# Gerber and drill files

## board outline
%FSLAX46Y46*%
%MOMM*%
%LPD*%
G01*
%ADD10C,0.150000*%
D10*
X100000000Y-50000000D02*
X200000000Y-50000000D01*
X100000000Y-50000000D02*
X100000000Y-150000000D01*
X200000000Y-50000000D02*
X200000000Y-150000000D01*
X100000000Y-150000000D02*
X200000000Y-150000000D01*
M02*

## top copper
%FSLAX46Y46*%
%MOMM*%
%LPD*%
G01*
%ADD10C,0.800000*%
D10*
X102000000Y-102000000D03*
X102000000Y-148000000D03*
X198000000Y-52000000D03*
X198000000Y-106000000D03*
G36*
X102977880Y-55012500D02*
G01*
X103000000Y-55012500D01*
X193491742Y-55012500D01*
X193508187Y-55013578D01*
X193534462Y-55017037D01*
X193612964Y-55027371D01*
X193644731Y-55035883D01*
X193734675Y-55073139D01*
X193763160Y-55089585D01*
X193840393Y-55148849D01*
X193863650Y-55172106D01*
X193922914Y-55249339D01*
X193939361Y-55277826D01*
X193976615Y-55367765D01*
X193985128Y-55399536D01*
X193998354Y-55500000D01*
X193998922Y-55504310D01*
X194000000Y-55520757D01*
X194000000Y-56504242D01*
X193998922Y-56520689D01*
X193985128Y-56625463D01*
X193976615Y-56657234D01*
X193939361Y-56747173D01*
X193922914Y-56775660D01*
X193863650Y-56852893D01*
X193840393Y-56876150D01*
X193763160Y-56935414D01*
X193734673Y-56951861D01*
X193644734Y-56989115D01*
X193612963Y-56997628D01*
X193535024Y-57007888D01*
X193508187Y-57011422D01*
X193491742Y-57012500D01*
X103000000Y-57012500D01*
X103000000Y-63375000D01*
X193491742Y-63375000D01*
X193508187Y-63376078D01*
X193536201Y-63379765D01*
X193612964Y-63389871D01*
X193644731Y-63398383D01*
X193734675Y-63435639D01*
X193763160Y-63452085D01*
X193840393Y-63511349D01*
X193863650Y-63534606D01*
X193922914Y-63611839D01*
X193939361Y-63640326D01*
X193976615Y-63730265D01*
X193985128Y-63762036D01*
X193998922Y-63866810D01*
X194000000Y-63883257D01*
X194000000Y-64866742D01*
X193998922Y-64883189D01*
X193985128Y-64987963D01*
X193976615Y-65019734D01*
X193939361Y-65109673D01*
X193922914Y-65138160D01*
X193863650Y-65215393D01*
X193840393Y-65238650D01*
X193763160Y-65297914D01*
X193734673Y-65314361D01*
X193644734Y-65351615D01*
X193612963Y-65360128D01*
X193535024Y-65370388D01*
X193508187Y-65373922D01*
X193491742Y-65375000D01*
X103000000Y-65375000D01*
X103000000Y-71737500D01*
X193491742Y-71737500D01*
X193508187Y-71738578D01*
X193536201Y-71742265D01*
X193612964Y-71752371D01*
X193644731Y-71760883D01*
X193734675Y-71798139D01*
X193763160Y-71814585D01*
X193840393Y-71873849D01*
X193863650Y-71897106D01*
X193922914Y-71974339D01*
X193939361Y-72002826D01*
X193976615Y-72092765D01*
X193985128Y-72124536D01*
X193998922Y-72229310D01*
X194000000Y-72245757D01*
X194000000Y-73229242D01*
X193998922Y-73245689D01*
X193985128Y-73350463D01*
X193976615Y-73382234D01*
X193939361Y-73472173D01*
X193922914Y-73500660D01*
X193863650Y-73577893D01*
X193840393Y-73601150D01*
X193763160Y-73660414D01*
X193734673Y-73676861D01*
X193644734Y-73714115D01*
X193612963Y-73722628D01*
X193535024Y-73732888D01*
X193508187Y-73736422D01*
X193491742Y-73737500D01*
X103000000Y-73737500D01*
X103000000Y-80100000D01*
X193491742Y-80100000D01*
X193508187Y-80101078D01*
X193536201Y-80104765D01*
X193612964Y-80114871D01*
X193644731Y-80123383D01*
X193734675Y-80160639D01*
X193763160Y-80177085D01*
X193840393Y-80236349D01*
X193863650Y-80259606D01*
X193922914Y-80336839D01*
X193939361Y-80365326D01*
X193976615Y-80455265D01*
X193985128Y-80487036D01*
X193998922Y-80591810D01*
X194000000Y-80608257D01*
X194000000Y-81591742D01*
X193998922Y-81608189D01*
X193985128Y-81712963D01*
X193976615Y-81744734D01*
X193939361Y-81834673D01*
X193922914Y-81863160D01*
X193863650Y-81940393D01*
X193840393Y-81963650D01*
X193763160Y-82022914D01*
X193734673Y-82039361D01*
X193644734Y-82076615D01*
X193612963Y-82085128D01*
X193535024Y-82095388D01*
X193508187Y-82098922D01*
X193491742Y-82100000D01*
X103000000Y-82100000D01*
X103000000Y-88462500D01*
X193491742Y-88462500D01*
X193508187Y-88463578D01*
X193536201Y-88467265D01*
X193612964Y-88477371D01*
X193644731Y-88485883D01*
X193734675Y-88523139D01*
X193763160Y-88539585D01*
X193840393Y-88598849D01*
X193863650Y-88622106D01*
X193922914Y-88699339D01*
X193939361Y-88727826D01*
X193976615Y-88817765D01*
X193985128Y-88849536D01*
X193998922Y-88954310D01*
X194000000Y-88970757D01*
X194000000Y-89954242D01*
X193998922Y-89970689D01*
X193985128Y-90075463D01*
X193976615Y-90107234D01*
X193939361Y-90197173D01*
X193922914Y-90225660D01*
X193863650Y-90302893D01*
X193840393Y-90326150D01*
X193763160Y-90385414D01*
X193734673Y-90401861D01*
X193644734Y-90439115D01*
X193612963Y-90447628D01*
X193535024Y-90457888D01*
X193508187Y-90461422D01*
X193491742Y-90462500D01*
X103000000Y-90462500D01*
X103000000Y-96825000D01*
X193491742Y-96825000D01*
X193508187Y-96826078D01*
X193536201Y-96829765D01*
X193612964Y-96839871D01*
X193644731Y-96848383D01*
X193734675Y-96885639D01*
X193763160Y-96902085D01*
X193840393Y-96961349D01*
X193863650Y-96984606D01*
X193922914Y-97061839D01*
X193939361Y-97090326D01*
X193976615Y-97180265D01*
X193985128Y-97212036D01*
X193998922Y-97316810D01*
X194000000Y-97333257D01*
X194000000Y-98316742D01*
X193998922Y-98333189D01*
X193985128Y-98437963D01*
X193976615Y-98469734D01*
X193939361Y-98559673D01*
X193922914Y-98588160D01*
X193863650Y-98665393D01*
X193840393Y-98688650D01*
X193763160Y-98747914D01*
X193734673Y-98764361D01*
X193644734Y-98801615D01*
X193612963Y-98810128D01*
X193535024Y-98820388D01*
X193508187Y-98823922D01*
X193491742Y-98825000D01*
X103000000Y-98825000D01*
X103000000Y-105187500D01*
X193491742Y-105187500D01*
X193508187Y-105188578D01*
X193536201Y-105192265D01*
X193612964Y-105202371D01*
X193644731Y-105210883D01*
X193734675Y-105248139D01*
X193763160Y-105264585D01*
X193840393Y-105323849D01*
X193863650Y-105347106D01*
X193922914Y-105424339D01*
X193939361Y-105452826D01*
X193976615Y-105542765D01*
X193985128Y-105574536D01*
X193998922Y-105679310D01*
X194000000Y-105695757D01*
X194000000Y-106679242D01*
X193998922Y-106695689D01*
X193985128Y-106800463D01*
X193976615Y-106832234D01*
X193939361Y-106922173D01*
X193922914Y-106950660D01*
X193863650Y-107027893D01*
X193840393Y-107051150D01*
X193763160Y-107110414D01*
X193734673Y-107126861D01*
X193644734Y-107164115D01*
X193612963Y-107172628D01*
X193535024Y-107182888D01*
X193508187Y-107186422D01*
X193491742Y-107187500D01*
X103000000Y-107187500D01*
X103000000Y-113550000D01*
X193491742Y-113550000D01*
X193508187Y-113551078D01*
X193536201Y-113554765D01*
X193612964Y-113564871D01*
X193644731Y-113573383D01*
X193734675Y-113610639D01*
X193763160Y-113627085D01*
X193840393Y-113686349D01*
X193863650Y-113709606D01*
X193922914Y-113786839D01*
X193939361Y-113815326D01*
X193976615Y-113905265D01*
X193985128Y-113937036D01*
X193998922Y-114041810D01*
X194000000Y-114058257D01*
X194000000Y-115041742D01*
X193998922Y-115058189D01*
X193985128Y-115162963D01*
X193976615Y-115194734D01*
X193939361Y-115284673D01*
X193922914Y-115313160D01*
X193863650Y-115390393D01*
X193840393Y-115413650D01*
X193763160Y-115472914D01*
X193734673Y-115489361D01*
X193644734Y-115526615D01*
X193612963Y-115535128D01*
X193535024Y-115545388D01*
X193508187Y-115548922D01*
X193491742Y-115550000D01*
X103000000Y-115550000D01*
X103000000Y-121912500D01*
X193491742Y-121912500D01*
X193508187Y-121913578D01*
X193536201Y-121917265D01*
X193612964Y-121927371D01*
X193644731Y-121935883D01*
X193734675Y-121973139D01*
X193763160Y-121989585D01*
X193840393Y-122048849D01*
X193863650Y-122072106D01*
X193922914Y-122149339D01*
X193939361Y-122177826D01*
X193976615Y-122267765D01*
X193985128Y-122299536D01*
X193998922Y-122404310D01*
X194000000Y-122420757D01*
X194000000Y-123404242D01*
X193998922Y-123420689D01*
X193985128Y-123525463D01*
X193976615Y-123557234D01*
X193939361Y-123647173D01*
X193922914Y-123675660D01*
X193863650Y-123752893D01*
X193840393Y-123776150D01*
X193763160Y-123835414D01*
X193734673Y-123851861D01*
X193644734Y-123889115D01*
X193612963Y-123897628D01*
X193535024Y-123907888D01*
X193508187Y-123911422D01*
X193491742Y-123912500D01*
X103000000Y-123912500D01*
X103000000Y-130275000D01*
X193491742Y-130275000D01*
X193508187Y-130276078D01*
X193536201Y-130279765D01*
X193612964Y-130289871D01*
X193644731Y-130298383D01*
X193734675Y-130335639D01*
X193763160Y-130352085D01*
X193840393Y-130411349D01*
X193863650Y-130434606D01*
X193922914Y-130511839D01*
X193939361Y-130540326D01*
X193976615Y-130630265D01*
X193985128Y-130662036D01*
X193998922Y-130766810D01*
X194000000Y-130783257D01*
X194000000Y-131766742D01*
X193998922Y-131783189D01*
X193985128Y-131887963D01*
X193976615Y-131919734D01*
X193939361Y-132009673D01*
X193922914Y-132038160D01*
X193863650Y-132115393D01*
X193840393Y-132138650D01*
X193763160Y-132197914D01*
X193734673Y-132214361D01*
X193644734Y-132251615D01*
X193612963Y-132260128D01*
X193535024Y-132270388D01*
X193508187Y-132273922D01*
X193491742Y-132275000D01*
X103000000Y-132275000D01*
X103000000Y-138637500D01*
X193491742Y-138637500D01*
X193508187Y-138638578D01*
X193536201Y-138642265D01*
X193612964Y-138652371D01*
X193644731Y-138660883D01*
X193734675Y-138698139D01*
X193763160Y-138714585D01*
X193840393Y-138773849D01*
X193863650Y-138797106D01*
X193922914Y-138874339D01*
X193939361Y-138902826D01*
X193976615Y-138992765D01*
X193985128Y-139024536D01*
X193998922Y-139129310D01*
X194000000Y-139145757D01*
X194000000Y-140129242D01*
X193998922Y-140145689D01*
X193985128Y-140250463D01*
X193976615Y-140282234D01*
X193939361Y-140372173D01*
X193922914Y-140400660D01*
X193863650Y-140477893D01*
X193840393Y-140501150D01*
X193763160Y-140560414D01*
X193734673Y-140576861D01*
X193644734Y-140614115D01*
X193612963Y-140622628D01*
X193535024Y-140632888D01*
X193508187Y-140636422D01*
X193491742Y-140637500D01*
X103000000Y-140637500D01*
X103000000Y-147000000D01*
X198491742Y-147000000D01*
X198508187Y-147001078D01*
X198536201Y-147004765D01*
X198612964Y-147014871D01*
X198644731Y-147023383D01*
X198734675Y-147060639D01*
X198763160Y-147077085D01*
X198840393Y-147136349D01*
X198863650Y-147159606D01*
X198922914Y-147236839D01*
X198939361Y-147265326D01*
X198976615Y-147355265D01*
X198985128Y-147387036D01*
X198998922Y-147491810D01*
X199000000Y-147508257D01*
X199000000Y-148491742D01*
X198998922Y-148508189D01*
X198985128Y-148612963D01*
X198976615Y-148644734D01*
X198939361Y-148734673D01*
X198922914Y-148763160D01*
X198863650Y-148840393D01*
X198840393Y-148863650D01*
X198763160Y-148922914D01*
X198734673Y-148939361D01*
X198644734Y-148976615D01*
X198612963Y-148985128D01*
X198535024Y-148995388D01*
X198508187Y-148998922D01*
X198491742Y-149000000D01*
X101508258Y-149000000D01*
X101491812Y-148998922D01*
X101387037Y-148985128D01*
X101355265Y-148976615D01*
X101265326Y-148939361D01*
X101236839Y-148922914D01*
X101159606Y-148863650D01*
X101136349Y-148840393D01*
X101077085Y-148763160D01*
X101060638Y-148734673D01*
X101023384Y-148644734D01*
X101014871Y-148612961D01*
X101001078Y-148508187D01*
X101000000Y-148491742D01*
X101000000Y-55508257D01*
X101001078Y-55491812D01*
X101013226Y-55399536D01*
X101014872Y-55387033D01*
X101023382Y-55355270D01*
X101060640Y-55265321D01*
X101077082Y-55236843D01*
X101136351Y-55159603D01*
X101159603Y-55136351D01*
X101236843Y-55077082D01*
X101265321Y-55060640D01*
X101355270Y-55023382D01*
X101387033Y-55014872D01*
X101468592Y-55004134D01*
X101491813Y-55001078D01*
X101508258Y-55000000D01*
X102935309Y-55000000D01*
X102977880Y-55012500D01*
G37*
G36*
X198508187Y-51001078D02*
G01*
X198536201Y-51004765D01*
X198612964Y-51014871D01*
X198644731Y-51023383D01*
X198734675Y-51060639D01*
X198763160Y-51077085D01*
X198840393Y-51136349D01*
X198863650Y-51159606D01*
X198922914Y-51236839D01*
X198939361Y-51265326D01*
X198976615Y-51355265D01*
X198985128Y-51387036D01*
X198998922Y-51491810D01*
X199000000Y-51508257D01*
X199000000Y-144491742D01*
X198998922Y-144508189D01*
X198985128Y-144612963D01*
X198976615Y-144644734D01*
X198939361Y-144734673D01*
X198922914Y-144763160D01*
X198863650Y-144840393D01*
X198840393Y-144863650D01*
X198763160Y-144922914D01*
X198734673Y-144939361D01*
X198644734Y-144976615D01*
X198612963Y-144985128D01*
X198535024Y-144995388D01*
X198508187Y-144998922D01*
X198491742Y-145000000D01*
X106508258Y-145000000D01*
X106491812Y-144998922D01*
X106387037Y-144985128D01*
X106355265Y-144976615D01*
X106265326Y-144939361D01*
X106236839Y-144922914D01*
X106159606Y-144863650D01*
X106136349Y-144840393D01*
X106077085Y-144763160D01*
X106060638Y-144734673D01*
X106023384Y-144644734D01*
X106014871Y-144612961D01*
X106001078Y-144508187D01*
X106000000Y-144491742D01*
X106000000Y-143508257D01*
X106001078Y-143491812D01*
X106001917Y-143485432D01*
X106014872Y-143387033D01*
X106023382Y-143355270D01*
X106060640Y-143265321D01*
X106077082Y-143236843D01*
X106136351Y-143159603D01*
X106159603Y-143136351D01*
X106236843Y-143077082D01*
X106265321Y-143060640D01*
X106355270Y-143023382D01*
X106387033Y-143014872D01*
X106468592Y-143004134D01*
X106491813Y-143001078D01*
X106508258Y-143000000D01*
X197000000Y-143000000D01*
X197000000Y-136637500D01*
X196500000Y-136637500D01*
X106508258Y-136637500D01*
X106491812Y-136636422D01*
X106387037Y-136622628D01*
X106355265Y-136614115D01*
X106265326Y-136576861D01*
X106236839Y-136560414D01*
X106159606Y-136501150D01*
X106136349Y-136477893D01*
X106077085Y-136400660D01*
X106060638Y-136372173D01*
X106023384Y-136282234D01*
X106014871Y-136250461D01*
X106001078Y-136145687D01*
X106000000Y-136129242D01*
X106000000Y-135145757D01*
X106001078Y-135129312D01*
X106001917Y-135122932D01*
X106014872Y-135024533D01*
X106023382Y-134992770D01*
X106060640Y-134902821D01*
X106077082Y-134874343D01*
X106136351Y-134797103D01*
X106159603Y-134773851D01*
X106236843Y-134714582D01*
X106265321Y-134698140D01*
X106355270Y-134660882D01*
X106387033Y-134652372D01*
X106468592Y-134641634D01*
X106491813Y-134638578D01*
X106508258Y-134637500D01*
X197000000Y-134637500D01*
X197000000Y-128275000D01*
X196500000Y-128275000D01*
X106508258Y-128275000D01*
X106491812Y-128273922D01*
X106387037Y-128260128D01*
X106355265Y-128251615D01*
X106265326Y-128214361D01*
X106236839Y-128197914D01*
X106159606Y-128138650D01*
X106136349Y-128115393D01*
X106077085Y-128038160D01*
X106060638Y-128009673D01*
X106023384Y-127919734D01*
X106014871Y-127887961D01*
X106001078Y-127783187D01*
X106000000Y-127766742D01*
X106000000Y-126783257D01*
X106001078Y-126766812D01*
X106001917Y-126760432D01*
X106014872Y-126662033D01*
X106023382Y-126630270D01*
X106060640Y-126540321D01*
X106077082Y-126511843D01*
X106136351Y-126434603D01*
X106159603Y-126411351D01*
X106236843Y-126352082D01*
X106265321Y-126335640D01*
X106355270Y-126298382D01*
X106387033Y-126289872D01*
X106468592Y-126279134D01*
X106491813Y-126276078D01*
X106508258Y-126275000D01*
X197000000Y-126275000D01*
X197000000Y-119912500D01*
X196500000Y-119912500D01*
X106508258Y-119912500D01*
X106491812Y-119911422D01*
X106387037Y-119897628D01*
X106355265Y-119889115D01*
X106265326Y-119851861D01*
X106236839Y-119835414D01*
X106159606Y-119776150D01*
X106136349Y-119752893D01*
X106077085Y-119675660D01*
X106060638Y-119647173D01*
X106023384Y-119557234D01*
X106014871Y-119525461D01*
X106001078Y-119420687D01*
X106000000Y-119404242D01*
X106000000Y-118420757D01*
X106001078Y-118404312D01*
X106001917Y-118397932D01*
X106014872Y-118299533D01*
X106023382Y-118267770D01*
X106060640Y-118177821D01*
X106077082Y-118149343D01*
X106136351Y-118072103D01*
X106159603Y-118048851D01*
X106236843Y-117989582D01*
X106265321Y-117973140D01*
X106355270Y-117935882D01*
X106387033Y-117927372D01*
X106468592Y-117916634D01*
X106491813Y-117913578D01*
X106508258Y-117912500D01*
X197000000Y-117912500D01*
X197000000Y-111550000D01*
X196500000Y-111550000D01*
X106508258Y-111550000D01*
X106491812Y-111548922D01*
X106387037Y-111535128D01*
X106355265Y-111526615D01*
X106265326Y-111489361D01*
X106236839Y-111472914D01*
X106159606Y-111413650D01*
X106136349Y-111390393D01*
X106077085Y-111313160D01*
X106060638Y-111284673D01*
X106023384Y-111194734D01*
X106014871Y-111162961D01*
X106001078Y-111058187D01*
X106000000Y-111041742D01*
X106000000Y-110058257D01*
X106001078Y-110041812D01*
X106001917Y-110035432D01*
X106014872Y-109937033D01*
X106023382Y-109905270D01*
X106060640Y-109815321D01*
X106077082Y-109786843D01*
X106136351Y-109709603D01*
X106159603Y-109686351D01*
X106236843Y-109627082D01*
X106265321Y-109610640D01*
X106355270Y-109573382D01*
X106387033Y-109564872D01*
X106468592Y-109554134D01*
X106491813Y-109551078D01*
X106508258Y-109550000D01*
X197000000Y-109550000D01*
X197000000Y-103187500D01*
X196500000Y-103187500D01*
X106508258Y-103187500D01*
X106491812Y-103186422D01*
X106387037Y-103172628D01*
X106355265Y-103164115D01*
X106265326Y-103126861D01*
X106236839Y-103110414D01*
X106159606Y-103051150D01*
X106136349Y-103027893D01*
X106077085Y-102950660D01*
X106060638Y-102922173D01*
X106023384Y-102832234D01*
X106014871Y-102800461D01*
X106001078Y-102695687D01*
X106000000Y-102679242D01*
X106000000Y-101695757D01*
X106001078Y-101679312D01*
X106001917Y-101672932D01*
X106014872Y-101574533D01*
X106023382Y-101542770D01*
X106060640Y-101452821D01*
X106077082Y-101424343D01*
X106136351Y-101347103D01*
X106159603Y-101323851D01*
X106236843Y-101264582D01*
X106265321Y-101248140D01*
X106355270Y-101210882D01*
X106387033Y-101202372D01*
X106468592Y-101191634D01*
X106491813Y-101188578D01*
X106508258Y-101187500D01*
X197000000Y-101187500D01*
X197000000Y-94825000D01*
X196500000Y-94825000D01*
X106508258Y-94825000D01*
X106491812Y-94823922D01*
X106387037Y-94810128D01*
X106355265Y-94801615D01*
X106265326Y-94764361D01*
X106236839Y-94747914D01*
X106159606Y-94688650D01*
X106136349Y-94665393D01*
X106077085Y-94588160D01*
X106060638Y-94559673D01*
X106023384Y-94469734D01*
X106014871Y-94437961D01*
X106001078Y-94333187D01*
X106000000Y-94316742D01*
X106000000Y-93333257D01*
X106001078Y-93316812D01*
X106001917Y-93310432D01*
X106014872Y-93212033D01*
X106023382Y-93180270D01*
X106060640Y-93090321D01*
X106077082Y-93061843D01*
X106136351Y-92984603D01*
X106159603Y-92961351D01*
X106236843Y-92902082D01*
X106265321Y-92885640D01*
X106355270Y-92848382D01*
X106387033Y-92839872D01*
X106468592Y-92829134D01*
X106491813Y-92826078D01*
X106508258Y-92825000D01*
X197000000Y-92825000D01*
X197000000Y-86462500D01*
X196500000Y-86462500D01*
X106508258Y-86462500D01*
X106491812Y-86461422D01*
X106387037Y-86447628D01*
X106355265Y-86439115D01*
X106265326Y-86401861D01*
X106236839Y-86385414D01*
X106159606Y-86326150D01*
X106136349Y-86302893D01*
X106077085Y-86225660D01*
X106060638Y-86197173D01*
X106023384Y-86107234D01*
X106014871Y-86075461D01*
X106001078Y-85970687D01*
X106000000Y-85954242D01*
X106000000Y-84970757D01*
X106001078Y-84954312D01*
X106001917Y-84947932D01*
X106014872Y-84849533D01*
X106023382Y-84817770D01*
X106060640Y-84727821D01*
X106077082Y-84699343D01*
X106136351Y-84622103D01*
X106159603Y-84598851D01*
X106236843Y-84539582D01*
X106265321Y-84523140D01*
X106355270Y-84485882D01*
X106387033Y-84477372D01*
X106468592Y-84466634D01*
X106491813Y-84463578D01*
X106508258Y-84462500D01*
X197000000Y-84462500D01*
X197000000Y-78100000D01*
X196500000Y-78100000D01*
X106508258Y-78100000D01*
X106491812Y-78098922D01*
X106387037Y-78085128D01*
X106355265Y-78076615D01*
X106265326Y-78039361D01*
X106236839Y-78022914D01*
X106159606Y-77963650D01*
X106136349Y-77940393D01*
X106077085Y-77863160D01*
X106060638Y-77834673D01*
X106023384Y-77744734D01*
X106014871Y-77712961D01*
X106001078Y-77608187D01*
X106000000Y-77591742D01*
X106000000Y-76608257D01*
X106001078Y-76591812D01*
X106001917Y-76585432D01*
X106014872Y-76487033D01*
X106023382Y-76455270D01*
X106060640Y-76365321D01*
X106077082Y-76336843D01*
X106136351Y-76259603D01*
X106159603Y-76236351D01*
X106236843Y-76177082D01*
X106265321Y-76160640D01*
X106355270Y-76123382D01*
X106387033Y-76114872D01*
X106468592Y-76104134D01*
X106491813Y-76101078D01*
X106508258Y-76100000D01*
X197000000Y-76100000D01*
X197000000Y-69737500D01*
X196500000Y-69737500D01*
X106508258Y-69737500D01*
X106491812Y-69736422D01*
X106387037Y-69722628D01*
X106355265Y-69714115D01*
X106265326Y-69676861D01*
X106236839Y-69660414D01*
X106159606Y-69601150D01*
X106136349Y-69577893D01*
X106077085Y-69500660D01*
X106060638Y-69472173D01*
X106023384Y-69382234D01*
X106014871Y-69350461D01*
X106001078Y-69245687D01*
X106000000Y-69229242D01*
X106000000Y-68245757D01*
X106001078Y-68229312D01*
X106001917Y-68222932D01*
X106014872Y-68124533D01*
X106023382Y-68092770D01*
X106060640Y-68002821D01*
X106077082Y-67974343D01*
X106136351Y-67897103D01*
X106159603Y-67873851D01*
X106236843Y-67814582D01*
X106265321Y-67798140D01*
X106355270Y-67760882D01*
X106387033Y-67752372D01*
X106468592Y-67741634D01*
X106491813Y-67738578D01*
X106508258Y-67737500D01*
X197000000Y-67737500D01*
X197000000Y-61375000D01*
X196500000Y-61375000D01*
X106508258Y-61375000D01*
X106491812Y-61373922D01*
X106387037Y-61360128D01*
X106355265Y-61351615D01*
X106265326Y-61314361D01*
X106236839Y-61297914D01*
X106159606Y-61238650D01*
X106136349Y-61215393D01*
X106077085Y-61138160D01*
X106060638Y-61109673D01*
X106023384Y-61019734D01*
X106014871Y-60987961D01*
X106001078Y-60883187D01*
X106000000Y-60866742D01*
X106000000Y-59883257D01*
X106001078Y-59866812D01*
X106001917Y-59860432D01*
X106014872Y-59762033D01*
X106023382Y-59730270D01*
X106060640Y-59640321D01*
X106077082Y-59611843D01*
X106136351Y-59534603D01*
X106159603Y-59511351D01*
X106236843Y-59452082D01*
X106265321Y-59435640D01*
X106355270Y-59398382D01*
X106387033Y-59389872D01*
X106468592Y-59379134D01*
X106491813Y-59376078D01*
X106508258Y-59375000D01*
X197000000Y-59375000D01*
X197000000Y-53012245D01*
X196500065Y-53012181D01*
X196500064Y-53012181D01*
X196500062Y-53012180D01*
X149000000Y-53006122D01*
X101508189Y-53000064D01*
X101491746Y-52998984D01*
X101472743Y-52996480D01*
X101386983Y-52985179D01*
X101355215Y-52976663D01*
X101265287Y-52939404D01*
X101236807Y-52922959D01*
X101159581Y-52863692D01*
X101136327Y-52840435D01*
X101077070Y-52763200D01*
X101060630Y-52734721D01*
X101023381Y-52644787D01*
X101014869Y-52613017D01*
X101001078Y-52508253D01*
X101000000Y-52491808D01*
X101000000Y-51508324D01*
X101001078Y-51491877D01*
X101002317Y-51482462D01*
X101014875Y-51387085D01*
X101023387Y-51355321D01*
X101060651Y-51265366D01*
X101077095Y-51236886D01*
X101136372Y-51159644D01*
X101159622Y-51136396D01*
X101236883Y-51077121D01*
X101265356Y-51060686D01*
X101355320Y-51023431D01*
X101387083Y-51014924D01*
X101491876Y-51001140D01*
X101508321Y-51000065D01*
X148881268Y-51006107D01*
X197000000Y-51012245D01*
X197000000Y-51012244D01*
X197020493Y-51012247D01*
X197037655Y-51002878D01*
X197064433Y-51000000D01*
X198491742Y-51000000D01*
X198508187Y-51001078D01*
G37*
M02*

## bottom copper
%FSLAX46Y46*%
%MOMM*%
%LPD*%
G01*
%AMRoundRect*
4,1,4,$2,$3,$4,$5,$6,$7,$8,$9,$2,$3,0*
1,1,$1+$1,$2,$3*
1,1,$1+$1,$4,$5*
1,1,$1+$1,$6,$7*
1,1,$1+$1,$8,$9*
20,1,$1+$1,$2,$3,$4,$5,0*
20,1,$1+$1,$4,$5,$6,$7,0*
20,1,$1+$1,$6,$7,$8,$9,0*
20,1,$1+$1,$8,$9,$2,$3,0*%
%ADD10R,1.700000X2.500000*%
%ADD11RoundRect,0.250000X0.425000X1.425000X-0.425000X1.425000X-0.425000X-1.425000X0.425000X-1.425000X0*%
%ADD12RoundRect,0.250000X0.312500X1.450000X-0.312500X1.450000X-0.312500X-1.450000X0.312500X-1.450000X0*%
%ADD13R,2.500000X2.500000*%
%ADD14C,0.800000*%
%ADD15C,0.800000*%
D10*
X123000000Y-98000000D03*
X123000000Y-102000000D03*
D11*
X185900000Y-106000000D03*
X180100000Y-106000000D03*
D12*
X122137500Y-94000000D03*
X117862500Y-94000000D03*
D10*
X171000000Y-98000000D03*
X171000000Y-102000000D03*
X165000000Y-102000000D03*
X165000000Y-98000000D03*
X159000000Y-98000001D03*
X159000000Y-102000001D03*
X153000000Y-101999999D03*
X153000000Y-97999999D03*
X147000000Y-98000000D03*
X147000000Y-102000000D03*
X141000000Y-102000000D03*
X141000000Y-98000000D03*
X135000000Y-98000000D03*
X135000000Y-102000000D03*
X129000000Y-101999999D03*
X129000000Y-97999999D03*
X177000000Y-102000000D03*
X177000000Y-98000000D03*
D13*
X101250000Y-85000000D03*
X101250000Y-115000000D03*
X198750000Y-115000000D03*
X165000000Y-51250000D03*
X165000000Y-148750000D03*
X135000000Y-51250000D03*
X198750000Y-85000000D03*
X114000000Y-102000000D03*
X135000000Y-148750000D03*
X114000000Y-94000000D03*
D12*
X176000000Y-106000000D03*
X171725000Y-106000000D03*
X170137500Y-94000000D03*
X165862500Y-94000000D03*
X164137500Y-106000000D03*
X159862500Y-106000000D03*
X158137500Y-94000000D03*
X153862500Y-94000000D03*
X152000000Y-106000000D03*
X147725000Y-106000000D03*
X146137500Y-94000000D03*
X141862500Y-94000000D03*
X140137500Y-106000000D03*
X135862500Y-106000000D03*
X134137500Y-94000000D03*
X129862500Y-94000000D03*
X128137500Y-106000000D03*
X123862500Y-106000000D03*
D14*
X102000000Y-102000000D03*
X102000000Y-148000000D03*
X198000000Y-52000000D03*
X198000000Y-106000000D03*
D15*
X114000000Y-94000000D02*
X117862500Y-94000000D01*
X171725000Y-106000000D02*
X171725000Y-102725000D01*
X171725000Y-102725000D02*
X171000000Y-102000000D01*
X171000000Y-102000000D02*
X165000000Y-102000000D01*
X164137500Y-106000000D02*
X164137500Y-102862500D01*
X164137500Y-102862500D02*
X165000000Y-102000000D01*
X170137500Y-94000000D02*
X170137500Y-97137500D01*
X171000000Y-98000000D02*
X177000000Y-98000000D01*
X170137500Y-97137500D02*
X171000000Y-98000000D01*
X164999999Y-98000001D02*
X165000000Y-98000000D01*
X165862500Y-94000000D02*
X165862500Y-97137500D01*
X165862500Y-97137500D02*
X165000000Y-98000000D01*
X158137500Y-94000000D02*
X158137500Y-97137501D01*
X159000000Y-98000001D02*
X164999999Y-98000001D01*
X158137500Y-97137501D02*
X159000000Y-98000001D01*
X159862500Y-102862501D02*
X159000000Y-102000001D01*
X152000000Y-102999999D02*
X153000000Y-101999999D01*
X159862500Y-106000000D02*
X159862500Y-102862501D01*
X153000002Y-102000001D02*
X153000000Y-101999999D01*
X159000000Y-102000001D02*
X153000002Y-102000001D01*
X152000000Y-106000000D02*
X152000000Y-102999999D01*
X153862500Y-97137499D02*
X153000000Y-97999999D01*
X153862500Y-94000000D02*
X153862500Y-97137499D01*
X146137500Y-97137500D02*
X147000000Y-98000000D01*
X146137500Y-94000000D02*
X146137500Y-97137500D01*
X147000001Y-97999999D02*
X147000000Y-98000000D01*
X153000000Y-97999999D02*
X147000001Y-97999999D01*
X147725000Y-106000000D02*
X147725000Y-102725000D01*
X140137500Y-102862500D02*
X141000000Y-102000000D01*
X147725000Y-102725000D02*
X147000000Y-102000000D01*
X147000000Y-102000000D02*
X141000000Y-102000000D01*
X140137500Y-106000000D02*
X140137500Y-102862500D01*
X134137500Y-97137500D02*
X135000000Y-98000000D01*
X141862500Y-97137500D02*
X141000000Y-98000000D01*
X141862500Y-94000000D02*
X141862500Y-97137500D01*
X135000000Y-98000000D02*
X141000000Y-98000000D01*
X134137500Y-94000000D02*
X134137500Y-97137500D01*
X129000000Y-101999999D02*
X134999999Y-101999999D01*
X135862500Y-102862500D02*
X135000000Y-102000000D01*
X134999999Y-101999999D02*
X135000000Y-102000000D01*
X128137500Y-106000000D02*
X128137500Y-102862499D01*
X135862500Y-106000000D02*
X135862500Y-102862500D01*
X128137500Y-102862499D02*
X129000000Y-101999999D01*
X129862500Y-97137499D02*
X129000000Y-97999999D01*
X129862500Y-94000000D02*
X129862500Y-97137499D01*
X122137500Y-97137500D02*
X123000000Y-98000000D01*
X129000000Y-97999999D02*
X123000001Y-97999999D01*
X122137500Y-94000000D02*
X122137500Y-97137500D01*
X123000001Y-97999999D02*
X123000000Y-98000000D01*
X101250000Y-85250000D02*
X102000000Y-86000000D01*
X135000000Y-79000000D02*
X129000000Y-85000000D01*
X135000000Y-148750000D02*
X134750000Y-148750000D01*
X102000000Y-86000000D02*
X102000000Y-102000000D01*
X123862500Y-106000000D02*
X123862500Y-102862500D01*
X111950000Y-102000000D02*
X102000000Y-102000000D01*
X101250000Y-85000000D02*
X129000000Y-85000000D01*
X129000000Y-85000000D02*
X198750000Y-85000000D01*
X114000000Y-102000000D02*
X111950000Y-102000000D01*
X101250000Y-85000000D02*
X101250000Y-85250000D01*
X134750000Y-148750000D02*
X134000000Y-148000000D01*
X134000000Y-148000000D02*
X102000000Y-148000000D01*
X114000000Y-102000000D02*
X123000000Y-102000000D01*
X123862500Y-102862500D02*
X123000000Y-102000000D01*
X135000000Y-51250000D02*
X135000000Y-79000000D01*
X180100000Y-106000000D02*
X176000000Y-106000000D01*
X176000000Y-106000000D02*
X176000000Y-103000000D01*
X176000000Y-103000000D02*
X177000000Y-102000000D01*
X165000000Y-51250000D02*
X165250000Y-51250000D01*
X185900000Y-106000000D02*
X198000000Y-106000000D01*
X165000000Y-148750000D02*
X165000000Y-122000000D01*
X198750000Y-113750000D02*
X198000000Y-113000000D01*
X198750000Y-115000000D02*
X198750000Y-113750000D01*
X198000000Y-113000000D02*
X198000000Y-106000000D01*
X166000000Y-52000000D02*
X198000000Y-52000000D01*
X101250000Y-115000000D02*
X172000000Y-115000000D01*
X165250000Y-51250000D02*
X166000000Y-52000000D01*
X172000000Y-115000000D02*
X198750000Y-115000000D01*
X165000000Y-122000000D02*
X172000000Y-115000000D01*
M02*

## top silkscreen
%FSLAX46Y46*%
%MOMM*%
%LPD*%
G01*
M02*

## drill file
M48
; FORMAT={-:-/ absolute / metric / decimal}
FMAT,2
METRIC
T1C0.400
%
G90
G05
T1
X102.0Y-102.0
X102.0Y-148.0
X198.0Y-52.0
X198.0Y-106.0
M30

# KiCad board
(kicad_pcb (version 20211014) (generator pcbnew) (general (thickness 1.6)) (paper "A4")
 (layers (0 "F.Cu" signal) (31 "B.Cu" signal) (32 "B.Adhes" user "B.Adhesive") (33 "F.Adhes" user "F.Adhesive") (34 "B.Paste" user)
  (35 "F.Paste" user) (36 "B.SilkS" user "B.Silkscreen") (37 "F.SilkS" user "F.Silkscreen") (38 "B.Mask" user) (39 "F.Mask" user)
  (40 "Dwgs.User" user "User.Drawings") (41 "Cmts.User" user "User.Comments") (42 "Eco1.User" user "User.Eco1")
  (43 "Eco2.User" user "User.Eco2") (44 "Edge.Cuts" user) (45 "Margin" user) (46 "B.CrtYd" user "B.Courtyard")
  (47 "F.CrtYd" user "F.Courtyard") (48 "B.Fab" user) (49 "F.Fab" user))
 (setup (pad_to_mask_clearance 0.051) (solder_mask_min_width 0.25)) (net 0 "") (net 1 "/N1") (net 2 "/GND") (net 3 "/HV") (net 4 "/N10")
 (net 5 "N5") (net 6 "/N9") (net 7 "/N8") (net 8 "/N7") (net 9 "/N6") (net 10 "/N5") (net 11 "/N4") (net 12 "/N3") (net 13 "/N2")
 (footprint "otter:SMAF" (layer "B.Cu") (at 123 100 -90)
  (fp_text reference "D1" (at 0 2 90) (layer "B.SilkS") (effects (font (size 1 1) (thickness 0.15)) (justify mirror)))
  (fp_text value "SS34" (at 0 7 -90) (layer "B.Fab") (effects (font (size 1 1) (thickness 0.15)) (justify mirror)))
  (pad "1" smd rect locked (at -2 0 270) (size 2.5 1.7) (layers "B.Cu" "B.Paste" "B.Mask") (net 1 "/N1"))
  (pad "2" smd rect locked (at 2 0 270) (size 2.5 1.7) (layers "B.Cu" "B.Paste" "B.Mask") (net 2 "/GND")))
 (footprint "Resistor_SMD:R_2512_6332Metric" (layer "B.Cu") (at 183 106 180)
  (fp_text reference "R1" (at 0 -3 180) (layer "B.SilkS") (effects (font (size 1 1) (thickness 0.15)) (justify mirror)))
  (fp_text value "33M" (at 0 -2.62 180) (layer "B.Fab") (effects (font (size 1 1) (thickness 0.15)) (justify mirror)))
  (pad "1" smd roundrect locked (at -2.9 0 180) (size 1.35 3.35) (layers "B.Cu" "B.Paste" "B.Mask") (roundrect_rratio 0.1851851852)
   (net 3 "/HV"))
  (pad "2" smd roundrect locked (at 2.9 0 180) (size 1.35 3.35) (layers "B.Cu" "B.Paste" "B.Mask") (roundrect_rratio 0.1851851852)
   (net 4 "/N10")))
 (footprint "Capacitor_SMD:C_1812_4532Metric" (layer "B.Cu") (at 120 94 180)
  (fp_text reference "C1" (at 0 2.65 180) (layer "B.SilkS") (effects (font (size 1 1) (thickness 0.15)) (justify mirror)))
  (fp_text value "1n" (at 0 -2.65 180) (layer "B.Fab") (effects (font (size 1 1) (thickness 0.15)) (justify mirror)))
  (pad "1" smd roundrect locked (at -2.1375 0 180) (size 1.125 3.4) (layers "B.Cu" "B.Paste" "B.Mask") (roundrect_rratio 0.2222222222)
   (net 1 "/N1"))
  (pad "2" smd roundrect locked (at 2.1375 0 180) (size 1.125 3.4) (layers "B.Cu" "B.Paste" "B.Mask") (roundrect_rratio 0.2222222222)
   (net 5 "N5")))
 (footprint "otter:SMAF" (layer "B.Cu") (at 171 100 -90)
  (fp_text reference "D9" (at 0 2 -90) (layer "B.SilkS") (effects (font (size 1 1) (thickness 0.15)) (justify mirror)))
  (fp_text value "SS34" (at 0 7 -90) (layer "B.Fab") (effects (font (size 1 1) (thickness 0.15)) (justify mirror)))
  (pad "1" smd rect locked (at -2 0 270) (size 2.5 1.7) (layers "B.Cu" "B.Paste" "B.Mask") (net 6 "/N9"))
  (pad "2" smd rect locked (at 2 0 270) (size 2.5 1.7) (layers "B.Cu" "B.Paste" "B.Mask") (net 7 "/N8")))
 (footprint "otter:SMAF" (layer "B.Cu") (at 165 100 90)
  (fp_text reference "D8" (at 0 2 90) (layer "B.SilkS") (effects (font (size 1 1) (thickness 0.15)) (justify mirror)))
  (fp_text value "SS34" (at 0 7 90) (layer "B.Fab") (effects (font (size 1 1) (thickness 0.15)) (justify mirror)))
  (pad "1" smd rect locked (at -2 0 90) (size 2.5 1.7) (layers "B.Cu" "B.Paste" "B.Mask") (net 7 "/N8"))
  (pad "2" smd rect locked (at 2 0 90) (size 2.5 1.7) (layers "B.Cu" "B.Paste" "B.Mask") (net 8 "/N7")))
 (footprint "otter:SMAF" (layer "B.Cu") (at 159 100.000001 -90)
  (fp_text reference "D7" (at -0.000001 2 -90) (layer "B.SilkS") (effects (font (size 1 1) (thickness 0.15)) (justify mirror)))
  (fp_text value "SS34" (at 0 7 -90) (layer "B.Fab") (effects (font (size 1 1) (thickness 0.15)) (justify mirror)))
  (pad "1" smd rect locked (at -2 0 270) (size 2.5 1.7) (layers "B.Cu" "B.Paste" "B.Mask") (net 8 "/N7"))
  (pad "2" smd rect locked (at 2 0 270) (size 2.5 1.7) (layers "B.Cu" "B.Paste" "B.Mask") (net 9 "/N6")))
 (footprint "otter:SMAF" (layer "B.Cu") (at 153 99.999999 90)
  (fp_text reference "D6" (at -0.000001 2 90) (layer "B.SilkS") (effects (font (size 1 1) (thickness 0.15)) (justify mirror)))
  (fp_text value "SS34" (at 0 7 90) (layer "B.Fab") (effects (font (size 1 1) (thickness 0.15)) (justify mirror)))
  (pad "1" smd rect locked (at -2 0 90) (size 2.5 1.7) (layers "B.Cu" "B.Paste" "B.Mask") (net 9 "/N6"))
  (pad "2" smd rect locked (at 2 0 90) (size 2.5 1.7) (layers "B.Cu" "B.Paste" "B.Mask") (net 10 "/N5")))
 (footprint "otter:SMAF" (layer "B.Cu") (at 147 100 -90)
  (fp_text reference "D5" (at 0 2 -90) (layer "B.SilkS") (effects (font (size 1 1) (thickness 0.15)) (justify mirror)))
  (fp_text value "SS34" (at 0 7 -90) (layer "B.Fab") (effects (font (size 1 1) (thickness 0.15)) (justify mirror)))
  (pad "1" smd rect locked (at -2 0 270) (size 2.5 1.7) (layers "B.Cu" "B.Paste" "B.Mask") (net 10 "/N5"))
  (pad "2" smd rect locked (at 2 0 270) (size 2.5 1.7) (layers "B.Cu" "B.Paste" "B.Mask") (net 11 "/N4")))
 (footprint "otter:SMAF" (layer "B.Cu") (at 141 100 90)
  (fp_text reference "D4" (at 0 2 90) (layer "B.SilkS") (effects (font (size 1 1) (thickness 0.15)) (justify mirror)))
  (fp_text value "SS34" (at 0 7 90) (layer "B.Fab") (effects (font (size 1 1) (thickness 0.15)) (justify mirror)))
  (pad "1" smd rect locked (at -2 0 90) (size 2.5 1.7) (layers "B.Cu" "B.Paste" "B.Mask") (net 11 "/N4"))
  (pad "2" smd rect locked (at 2 0 90) (size 2.5 1.7) (layers "B.Cu" "B.Paste" "B.Mask") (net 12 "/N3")))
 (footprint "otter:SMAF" (layer "B.Cu") (at 135 100 -90)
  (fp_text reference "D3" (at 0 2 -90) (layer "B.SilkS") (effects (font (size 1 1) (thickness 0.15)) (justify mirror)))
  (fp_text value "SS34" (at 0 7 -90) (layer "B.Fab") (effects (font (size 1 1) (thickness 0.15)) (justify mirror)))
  (pad "1" smd rect locked (at -2 0 270) (size 2.5 1.7) (layers "B.Cu" "B.Paste" "B.Mask") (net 12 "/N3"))
  (pad "2" smd rect locked (at 2 0 270) (size 2.5 1.7) (layers "B.Cu" "B.Paste" "B.Mask") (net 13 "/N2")))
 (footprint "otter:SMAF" (layer "B.Cu") (at 129 99.999999 90)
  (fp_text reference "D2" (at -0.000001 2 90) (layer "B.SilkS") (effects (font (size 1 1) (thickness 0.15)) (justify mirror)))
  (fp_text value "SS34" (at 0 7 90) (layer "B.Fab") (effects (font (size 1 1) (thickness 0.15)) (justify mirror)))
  (pad "1" smd rect locked (at -2 0 90) (size 2.5 1.7) (layers "B.Cu" "B.Paste" "B.Mask") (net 13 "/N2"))
  (pad "2" smd rect locked (at 2 0 90) (size 2.5 1.7) (layers "B.Cu" "B.Paste" "B.Mask") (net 1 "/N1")))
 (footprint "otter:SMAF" (layer "B.Cu") (at 177 100 90)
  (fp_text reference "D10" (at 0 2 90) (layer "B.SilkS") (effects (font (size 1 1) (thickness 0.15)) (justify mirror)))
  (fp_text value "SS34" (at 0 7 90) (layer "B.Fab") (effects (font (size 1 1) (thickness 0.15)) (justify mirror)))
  (pad "1" smd rect locked (at -2 0 90) (size 2.5 1.7) (layers "B.Cu" "B.Paste" "B.Mask") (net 4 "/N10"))
  (pad "2" smd rect locked (at 2 0 90) (size 2.5 1.7) (layers "B.Cu" "B.Paste" "B.Mask") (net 6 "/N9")))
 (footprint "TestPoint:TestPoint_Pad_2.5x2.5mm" (layer "B.Cu") (at 101.25 85 180)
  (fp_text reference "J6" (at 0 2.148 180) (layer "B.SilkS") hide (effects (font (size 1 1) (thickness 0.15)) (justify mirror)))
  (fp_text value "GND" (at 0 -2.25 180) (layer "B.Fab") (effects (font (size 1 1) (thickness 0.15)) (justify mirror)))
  (pad "1" smd rect locked (at 0 0 180) (size 2.5 2.5) (layers "B.Cu" "B.Mask") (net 2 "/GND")))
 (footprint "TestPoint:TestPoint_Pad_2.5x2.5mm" (layer "B.Cu") (at 101.25 115 180)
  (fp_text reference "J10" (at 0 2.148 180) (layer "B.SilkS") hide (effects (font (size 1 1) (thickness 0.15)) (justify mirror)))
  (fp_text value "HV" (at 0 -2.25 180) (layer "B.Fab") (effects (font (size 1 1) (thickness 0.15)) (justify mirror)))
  (pad "1" smd rect locked (at 0 0 180) (size 2.5 2.5) (layers "B.Cu" "B.Mask") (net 3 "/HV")))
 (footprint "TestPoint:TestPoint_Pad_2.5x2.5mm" (layer "B.Cu") (at 198.75 115 180)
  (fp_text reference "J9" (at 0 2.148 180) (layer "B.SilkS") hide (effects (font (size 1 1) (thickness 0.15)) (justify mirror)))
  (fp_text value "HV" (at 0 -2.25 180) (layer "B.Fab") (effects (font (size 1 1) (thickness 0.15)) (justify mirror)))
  (pad "1" smd rect locked (at 0 0 180) (size 2.5 2.5) (layers "B.Cu" "B.Mask") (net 3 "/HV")))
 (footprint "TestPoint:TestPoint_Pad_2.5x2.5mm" (layer "B.Cu") (at 165 51.25 180)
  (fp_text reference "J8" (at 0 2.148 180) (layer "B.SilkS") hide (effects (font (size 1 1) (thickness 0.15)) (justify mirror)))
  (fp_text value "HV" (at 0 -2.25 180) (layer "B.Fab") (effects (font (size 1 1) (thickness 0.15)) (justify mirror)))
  (pad "1" smd rect locked (at 0 0 180) (size 2.5 2.5) (layers "B.Cu" "B.Mask") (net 3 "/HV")))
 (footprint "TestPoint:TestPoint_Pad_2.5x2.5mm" (layer "B.Cu") (at 165 148.75 180)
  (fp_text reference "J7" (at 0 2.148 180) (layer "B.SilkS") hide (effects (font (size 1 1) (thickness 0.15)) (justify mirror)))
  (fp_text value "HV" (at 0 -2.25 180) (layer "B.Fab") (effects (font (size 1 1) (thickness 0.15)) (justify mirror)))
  (pad "1" smd rect locked (at 0 0 180) (size 2.5 2.5) (layers "B.Cu" "B.Mask") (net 3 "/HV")))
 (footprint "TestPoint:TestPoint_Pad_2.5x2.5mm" (layer "B.Cu") (at 135 51.25 180)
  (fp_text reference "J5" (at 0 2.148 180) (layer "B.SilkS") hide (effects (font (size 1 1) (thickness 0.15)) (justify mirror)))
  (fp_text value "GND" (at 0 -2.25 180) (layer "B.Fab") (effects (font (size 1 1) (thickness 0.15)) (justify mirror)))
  (pad "1" smd rect locked (at 0 0 180) (size 2.5 2.5) (layers "B.Cu" "B.Mask") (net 2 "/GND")))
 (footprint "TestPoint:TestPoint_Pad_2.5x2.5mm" (layer "B.Cu") (at 198.75 85 180)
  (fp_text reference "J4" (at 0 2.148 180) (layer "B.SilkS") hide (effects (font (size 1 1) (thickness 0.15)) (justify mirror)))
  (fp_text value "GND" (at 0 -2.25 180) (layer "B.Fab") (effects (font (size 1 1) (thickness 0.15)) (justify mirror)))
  (pad "1" smd rect locked (at 0 0 180) (size 2.5 2.5) (layers "B.Cu" "B.Mask") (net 2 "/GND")))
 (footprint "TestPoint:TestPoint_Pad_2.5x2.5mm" (layer "B.Cu") (at 114 102 180)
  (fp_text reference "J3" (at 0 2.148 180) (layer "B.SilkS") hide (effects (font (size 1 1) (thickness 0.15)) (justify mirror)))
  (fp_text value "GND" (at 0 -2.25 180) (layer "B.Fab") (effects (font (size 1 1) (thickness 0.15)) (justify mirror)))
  (pad "1" smd rect locked (at 0 0 180) (size 2.5 2.5) (layers "B.Cu" "B.Mask") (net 2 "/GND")))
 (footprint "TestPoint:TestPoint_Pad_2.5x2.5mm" (layer "B.Cu") (at 135 148.75 180)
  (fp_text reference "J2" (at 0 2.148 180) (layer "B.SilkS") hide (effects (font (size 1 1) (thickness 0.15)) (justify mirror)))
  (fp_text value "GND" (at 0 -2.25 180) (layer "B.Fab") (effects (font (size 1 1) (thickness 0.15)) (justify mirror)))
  (pad "1" smd rect locked (at 0 0 180) (size 2.5 2.5) (layers "B.Cu" "B.Mask") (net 2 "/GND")))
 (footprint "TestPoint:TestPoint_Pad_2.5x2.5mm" (layer "B.Cu") (at 114 94 180)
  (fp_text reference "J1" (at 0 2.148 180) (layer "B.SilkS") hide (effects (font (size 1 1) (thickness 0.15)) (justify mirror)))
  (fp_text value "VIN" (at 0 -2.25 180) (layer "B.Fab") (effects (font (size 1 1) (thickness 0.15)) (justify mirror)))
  (pad "1" smd rect locked (at 0 0 180) (size 2.5 2.5) (layers "B.Cu" "B.Mask") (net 5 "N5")))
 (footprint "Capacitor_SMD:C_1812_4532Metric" (layer "B.Cu") (at 173.8625 106 180)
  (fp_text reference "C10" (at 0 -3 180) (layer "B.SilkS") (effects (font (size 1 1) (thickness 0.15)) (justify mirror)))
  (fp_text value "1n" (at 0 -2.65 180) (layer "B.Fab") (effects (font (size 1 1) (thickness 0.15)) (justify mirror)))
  (pad "1" smd roundrect locked (at -2.1375 0 180) (size 1.125 3.4) (layers "B.Cu" "B.Paste" "B.Mask") (roundrect_rratio 0.2222222222)
   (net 4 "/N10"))
  (pad "2" smd roundrect locked (at 2.1375 0 180) (size 1.125 3.4) (layers "B.Cu" "B.Paste" "B.Mask") (roundrect_rratio 0.2222222222)
   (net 7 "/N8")))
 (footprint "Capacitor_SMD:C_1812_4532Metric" (layer "B.Cu") (at 168 94 180)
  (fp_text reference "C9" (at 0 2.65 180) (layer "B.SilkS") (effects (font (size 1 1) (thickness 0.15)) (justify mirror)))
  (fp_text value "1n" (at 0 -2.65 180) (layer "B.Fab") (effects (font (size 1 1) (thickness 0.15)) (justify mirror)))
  (pad "1" smd roundrect locked (at -2.1375 0 180) (size 1.125 3.4) (layers "B.Cu" "B.Paste" "B.Mask") (roundrect_rratio 0.2222222222)
   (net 6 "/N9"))
  (pad "2" smd roundrect locked (at 2.1375 0 180) (size 1.125 3.4) (layers "B.Cu" "B.Paste" "B.Mask") (roundrect_rratio 0.2222222222)
   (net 8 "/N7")))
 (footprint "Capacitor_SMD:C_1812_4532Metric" (layer "B.Cu") (at 162 106 180)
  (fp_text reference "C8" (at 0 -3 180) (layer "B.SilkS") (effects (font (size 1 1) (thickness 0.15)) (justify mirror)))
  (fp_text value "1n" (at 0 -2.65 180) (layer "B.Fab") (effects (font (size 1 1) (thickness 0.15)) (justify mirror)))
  (pad "1" smd roundrect locked (at -2.1375 0 180) (size 1.125 3.4) (layers "B.Cu" "B.Paste" "B.Mask") (roundrect_rratio 0.2222222222)
   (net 7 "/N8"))
  (pad "2" smd roundrect locked (at 2.1375 0 180) (size 1.125 3.4) (layers "B.Cu" "B.Paste" "B.Mask") (roundrect_rratio 0.2222222222)
   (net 9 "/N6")))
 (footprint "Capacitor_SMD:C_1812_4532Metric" (layer "B.Cu") (at 156 94 180)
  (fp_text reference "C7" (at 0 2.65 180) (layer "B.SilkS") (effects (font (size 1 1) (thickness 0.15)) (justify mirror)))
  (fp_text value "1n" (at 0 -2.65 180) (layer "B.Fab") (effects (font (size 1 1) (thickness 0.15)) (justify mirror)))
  (pad "1" smd roundrect locked (at -2.1375 0 180) (size 1.125 3.4) (layers "B.Cu" "B.Paste" "B.Mask") (roundrect_rratio 0.2222222222)
   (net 8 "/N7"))
  (pad "2" smd roundrect locked (at 2.1375 0 180) (size 1.125 3.4) (layers "B.Cu" "B.Paste" "B.Mask") (roundrect_rratio 0.2222222222)
   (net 10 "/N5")))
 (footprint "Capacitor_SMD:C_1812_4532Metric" (layer "B.Cu") (at 149.8625 106 180)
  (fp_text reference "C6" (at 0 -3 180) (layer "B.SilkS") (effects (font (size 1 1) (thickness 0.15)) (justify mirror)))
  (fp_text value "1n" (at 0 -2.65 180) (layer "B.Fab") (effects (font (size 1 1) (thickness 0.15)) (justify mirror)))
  (pad "1" smd roundrect locked (at -2.1375 0 180) (size 1.125 3.4) (layers "B.Cu" "B.Paste" "B.Mask") (roundrect_rratio 0.2222222222)
   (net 9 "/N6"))
  (pad "2" smd roundrect locked (at 2.1375 0 180) (size 1.125 3.4) (layers "B.Cu" "B.Paste" "B.Mask") (roundrect_rratio 0.2222222222)
   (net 11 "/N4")))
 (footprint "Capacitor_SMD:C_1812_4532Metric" (layer "B.Cu") (at 144 94 180)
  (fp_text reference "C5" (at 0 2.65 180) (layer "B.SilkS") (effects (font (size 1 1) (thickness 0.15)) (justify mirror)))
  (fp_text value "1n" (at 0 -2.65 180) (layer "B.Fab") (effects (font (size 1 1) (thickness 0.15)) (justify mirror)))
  (pad "1" smd roundrect locked (at -2.1375 0 180) (size 1.125 3.4) (layers "B.Cu" "B.Paste" "B.Mask") (roundrect_rratio 0.2222222222)
   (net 10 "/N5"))
  (pad "2" smd roundrect locked (at 2.1375 0 180) (size 1.125 3.4) (layers "B.Cu" "B.Paste" "B.Mask") (roundrect_rratio 0.2222222222)
   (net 12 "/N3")))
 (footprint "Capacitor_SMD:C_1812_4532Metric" (layer "B.Cu") (at 138 106 180)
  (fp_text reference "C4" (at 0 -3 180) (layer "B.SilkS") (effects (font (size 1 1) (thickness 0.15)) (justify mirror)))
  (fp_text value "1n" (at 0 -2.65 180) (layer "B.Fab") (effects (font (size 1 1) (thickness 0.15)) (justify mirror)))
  (pad "1" smd roundrect locked (at -2.1375 0 180) (size 1.125 3.4) (layers "B.Cu" "B.Paste" "B.Mask") (roundrect_rratio 0.2222222222)
   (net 11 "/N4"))
  (pad "2" smd roundrect locked (at 2.1375 0 180) (size 1.125 3.4) (layers "B.Cu" "B.Paste" "B.Mask") (roundrect_rratio 0.2222222222)
   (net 13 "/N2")))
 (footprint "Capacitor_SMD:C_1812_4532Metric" (layer "B.Cu") (at 132 94 180)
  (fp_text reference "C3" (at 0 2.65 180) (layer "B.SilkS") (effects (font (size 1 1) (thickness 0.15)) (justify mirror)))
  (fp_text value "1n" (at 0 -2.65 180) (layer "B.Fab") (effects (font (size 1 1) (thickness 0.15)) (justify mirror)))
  (pad "1" smd roundrect locked (at -2.1375 0 180) (size 1.125 3.4) (layers "B.Cu" "B.Paste" "B.Mask") (roundrect_rratio 0.2222222222)
   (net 12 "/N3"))
  (pad "2" smd roundrect locked (at 2.1375 0 180) (size 1.125 3.4) (layers "B.Cu" "B.Paste" "B.Mask") (roundrect_rratio 0.2222222222)
   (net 1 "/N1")))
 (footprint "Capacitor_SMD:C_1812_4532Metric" (layer "B.Cu") (at 126 106 180)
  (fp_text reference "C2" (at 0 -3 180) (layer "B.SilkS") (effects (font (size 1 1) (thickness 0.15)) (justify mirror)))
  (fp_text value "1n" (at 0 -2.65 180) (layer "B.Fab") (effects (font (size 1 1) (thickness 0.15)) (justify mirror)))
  (pad "1" smd roundrect locked (at -2.1375 0 180) (size 1.125 3.4) (layers "B.Cu" "B.Paste" "B.Mask") (roundrect_rratio 0.2222222222)
   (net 13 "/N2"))
  (pad "2" smd roundrect locked (at 2.1375 0 180) (size 1.125 3.4) (layers "B.Cu" "B.Paste" "B.Mask") (roundrect_rratio 0.2222222222)
   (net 2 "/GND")))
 (gr_line (start 100 50) (end 200 50) (layer "Edge.Cuts") (width 0.15))
 (gr_line (start 100 50) (end 100 150) (layer "Edge.Cuts") (width 0.15))
 (gr_line (start 200 50) (end 200 150) (layer "Edge.Cuts") (width 0.15))
 (gr_line (start 100 150) (end 200 150) (layer "Edge.Cuts") (width 0.15))
 (segment (start 114 94) (end 117.8625 94) (width 0.8) (layer "B.Cu") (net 5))
 (segment (start 171.725 106) (end 171.725 102.725) (width 0.8) (layer "B.Cu") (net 7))
 (segment (start 171.725 102.725) (end 171 102) (width 0.8) (layer "B.Cu") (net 7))
 (segment (start 171 102) (end 165 102) (width 0.8) (layer "B.Cu") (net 7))
 (segment (start 164.1375 106) (end 164.1375 102.8625) (width 0.8) (layer "B.Cu") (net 7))
 (segment (start 164.1375 102.8625) (end 165 102) (width 0.8) (layer "B.Cu") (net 7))
 (segment (start 170.1375 94) (end 170.1375 97.1375) (width 0.8) (layer "B.Cu") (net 6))
 (segment (start 171 98) (end 177 98) (width 0.8) (layer "B.Cu") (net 6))
 (segment (start 170.1375 97.1375) (end 171 98) (width 0.8) (layer "B.Cu") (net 6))
 (segment (start 164.999999 98.000001) (end 165 98) (width 0.8) (layer "B.Cu") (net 8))
 (segment (start 165.8625 94) (end 165.8625 97.1375) (width 0.8) (layer "B.Cu") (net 8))
 (segment (start 165.8625 97.1375) (end 165 98) (width 0.8) (layer "B.Cu") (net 8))
 (segment (start 158.1375 94) (end 158.1375 97.137501) (width 0.8) (layer "B.Cu") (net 8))
 (segment (start 159 98.000001) (end 164.999999 98.000001) (width 0.8) (layer "B.Cu") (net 8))
 (segment (start 158.1375 97.137501) (end 159 98.000001) (width 0.8) (layer "B.Cu") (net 8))
 (segment (start 159.8625 102.862501) (end 159 102.000001) (width 0.8) (layer "B.Cu") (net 9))
 (segment (start 152 102.999999) (end 153 101.999999) (width 0.8) (layer "B.Cu") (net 9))
 (segment (start 159.8625 106) (end 159.8625 102.862501) (width 0.8) (layer "B.Cu") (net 9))
 (segment (start 153.000002 102.000001) (end 153 101.999999) (width 0.8) (layer "B.Cu") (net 9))
 (segment (start 159 102.000001) (end 153.000002 102.000001) (width 0.8) (layer "B.Cu") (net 9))
 (segment (start 152 106) (end 152 102.999999) (width 0.8) (layer "B.Cu") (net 9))
 (segment (start 153.8625 97.137499) (end 153 97.999999) (width 0.8) (layer "B.Cu") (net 10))
 (segment (start 153.8625 94) (end 153.8625 97.137499) (width 0.8) (layer "B.Cu") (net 10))
 (segment (start 146.1375 97.1375) (end 147 98) (width 0.8) (layer "B.Cu") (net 10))
 (segment (start 146.1375 94) (end 146.1375 97.1375) (width 0.8) (layer "B.Cu") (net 10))
 (segment (start 147.000001 97.999999) (end 147 98) (width 0.8) (layer "B.Cu") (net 10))
 (segment (start 153 97.999999) (end 147.000001 97.999999) (width 0.8) (layer "B.Cu") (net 10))
 (segment (start 147.725 106) (end 147.725 102.725) (width 0.8) (layer "B.Cu") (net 11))
 (segment (start 140.1375 102.8625) (end 141 102) (width 0.8) (layer "B.Cu") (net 11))
 (segment (start 147.725 102.725) (end 147 102) (width 0.8) (layer "B.Cu") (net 11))
 (segment (start 147 102) (end 141 102) (width 0.8) (layer "B.Cu") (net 11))
 (segment (start 140.1375 106) (end 140.1375 102.8625) (width 0.8) (layer "B.Cu") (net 11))
 (segment (start 134.1375 97.1375) (end 135 98) (width 0.8) (layer "B.Cu") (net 12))
 (segment (start 141.8625 97.1375) (end 141 98) (width 0.8) (layer "B.Cu") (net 12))
 (segment (start 141.8625 94) (end 141.8625 97.1375) (width 0.8) (layer "B.Cu") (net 12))
 (segment (start 135 98) (end 141 98) (width 0.8) (layer "B.Cu") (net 12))
 (segment (start 134.1375 94) (end 134.1375 97.1375) (width 0.8) (layer "B.Cu") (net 12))
 (segment (start 129 101.999999) (end 134.999999 101.999999) (width 0.8) (layer "B.Cu") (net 13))
 (segment (start 135.8625 102.8625) (end 135 102) (width 0.8) (layer "B.Cu") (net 13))
 (segment (start 134.999999 101.999999) (end 135 102) (width 0.8) (layer "B.Cu") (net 13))
 (segment (start 128.1375 106) (end 128.1375 102.862499) (width 0.8) (layer "B.Cu") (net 13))
 (segment (start 135.8625 106) (end 135.8625 102.8625) (width 0.8) (layer "B.Cu") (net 13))
 (segment (start 128.1375 102.862499) (end 129 101.999999) (width 0.8) (layer "B.Cu") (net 13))
 (segment (start 129.8625 97.137499) (end 129 97.999999) (width 0.8) (layer "B.Cu") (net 1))
 (segment (start 129.8625 94) (end 129.8625 97.137499) (width 0.8) (layer "B.Cu") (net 1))
 (segment (start 122.1375 97.1375) (end 123 98) (width 0.8) (layer "B.Cu") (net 1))
 (segment (start 129 97.999999) (end 123.000001 97.999999) (width 0.8) (layer "B.Cu") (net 1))
 (segment (start 122.1375 94) (end 122.1375 97.1375) (width 0.8) (layer "B.Cu") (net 1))
 (segment (start 123.000001 97.999999) (end 123 98) (width 0.8) (layer "B.Cu") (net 1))
 (via (at 102 102) (size 0.8) (drill 0.4) (layers "F.Cu" "B.Cu") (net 2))
 (via (at 102 148) (size 0.8) (drill 0.4) (layers "F.Cu" "B.Cu") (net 2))
 (segment (start 101.25 85.25) (end 102 86) (width 0.8) (layer "B.Cu") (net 2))
 (segment (start 135 79) (end 129 85) (width 0.8) (layer "B.Cu") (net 2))
 (segment (start 135 148.75) (end 134.75 148.75) (width 0.8) (layer "B.Cu") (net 2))
 (segment (start 102 86) (end 102 102) (width 0.8) (layer "B.Cu") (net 2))
 (segment (start 123.8625 106) (end 123.8625 102.8625) (width 0.8) (layer "B.Cu") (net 2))
 (segment (start 111.95 102) (end 102 102) (width 0.8) (layer "B.Cu") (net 2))
 (segment (start 101.25 85) (end 129 85) (width 0.8) (layer "B.Cu") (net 2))
 (segment (start 129 85) (end 198.75 85) (width 0.8) (layer "B.Cu") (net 2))
 (segment (start 114 102) (end 111.95 102) (width 0.8) (layer "B.Cu") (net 2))
 (segment (start 101.25 85) (end 101.25 85.25) (width 0.8) (layer "B.Cu") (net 2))
 (segment (start 134.75 148.75) (end 134 148) (width 0.8) (layer "B.Cu") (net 2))
 (segment (start 134 148) (end 102 148) (width 0.8) (layer "B.Cu") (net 2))
 (segment (start 114 102) (end 123 102) (width 0.8) (layer "B.Cu") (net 2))
 (segment (start 123.8625 102.8625) (end 123 102) (width 0.8) (layer "B.Cu") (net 2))
 (segment (start 135 51.25) (end 135 79) (width 0.8) (layer "B.Cu") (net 2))
 (segment (start 180.1 106) (end 176 106) (width 0.8) (layer "B.Cu") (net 4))
 (segment (start 176 106) (end 176 103) (width 0.8) (layer "B.Cu") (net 4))
 (segment (start 176 103) (end 177 102) (width 0.8) (layer "B.Cu") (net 4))
 (via (at 198 52) (size 0.8) (drill 0.4) (layers "F.Cu" "B.Cu") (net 3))
 (via (at 198 106) (size 0.8) (drill 0.4) (layers "F.Cu" "B.Cu") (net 3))
 (segment (start 165 51.25) (end 165.25 51.25) (width 0.8) (layer "B.Cu") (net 3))
 (segment (start 185.9 106) (end 198 106) (width 0.8) (layer "B.Cu") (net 3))
 (segment (start 165 148.75) (end 165 122) (width 0.8) (layer "B.Cu") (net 3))
 (segment (start 198.75 113.75) (end 198 113) (width 0.8) (layer "B.Cu") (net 3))
 (segment (start 198.75 115) (end 198.75 113.75) (width 0.8) (layer "B.Cu") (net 3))
 (segment (start 198 113) (end 198 106) (width 0.8) (layer "B.Cu") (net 3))
 (segment (start 166 52) (end 198 52) (width 0.8) (layer "B.Cu") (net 3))
 (segment (start 101.25 115) (end 172 115) (width 0.8) (layer "B.Cu") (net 3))
 (segment (start 165.25 51.25) (end 166 52) (width 0.8) (layer "B.Cu") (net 3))
 (segment (start 172 115) (end 198.75 115) (width 0.8) (layer "B.Cu") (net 3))
 (segment (start 165 122) (end 172 115) (width 0.8) (layer "B.Cu") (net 3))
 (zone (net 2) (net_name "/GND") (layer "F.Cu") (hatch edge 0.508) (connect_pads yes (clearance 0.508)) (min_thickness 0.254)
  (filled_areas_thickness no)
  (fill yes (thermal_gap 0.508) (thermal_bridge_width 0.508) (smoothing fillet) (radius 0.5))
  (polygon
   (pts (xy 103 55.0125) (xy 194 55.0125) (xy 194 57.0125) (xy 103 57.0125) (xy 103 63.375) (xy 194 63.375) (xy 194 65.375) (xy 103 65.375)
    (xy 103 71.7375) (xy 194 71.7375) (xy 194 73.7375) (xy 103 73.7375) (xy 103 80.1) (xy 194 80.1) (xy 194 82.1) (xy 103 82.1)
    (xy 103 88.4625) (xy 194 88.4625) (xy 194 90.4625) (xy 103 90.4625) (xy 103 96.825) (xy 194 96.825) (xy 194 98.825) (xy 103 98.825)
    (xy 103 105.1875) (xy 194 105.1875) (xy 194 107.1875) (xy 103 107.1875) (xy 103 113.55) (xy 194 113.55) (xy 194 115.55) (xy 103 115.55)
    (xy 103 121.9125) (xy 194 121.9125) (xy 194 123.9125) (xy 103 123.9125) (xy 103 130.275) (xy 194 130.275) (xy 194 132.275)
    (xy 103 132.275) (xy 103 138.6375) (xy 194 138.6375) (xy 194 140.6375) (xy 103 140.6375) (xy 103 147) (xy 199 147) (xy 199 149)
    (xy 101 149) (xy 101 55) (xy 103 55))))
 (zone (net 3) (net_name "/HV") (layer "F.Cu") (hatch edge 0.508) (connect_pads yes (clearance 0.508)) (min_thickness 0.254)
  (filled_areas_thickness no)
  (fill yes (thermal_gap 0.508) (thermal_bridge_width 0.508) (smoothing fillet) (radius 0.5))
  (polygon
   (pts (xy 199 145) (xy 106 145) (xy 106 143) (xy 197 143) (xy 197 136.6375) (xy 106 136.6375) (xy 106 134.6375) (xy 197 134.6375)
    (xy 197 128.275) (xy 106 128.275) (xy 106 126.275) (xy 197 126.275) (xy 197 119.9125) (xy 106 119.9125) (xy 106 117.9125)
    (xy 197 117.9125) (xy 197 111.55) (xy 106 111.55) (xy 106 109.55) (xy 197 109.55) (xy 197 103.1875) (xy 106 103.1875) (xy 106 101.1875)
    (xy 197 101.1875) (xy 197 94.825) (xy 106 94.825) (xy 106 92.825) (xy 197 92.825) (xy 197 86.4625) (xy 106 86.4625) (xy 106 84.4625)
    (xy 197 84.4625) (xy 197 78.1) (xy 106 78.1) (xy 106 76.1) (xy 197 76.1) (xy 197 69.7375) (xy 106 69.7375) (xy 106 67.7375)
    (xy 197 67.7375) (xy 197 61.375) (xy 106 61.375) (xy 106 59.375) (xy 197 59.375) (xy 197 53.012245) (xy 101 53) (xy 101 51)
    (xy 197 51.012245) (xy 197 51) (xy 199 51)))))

